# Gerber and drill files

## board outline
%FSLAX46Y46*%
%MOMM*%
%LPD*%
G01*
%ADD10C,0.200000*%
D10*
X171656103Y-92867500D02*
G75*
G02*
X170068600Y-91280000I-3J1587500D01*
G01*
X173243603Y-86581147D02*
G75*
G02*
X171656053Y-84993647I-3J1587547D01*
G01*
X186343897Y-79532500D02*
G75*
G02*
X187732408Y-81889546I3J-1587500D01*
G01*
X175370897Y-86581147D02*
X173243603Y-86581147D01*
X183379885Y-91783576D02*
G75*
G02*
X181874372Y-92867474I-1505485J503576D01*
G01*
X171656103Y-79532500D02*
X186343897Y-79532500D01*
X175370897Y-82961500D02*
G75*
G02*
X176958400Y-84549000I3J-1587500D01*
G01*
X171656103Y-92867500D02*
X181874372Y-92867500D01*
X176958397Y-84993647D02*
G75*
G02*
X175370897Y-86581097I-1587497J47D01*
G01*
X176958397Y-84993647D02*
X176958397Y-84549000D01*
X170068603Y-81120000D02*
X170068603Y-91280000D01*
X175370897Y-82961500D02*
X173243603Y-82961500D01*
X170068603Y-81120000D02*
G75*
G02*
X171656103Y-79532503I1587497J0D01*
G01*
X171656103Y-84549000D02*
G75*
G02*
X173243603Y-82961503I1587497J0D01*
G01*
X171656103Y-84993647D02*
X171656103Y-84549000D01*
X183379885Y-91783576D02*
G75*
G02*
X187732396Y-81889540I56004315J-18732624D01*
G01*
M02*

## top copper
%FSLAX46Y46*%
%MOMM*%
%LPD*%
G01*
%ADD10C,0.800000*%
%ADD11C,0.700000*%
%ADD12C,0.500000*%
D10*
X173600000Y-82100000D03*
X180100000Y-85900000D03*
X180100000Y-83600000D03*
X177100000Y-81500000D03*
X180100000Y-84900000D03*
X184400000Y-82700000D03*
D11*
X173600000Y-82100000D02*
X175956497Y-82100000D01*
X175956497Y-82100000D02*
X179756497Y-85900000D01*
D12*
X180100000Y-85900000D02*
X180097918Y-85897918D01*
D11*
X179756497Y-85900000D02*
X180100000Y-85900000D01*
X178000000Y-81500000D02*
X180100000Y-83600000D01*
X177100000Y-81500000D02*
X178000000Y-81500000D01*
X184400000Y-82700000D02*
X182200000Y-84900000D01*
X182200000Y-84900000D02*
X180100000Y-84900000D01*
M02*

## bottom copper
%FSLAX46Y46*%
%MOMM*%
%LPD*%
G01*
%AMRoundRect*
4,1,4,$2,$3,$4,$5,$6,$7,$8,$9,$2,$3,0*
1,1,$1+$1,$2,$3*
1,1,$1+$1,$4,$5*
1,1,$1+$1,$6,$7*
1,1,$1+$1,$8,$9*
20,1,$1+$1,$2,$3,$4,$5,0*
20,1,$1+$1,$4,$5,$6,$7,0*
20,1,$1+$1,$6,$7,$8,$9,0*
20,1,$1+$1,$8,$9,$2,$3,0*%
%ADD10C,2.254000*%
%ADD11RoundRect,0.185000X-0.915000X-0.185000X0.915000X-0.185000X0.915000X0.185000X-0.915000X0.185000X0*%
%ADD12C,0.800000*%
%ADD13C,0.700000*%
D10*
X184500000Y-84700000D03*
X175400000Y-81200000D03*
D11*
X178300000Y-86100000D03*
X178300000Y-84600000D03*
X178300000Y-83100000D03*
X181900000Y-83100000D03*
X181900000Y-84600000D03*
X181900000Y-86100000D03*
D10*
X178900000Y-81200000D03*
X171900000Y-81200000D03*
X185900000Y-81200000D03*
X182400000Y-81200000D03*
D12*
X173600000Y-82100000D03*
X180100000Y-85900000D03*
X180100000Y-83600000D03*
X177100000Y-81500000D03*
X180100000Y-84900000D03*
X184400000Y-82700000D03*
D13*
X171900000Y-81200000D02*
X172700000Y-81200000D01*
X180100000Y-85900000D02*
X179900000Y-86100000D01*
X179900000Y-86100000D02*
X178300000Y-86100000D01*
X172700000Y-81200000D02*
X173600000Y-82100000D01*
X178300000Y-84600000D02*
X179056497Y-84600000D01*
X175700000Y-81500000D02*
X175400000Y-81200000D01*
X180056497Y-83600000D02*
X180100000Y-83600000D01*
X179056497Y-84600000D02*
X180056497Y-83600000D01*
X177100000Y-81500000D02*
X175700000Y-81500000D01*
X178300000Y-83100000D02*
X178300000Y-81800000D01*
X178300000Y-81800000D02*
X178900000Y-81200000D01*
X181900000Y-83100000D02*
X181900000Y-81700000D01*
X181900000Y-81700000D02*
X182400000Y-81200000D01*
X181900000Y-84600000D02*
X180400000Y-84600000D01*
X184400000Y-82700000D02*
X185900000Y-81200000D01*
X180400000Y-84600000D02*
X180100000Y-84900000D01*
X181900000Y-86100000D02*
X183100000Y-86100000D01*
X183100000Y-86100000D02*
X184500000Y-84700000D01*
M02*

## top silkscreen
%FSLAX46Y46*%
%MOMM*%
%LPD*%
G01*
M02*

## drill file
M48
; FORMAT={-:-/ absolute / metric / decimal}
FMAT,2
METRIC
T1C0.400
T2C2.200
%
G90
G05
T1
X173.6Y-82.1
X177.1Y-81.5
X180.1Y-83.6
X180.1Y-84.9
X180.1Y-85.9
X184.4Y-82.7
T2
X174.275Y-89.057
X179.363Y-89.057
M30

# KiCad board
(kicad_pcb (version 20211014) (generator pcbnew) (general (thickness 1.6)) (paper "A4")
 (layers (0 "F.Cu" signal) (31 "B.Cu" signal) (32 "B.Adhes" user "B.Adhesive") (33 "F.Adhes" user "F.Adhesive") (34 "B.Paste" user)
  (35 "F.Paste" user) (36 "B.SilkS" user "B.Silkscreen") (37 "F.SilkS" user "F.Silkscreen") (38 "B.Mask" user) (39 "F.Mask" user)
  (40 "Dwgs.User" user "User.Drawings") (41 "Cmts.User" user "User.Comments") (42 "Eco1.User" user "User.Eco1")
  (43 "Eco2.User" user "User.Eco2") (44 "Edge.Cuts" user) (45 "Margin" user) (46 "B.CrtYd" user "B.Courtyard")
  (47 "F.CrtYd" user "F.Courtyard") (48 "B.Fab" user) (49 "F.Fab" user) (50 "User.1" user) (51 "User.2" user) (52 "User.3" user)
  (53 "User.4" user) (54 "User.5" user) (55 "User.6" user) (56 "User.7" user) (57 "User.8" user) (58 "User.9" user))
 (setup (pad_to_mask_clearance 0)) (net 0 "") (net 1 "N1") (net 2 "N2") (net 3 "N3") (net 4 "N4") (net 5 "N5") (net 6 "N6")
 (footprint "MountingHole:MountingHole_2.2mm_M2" (layer "F.Cu") (at 179.362966 89.0575)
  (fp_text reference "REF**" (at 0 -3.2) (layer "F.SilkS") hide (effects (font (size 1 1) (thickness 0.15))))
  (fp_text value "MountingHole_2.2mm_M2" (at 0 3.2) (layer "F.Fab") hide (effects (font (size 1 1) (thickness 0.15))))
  (pad "" np_thru_hole circle (at 0 0) (size 2.2 2.2) (drill 2.2) (layers *.Cu *.Mask)))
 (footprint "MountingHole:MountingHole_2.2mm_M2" (layer "F.Cu") (at 174.275478 89.0575)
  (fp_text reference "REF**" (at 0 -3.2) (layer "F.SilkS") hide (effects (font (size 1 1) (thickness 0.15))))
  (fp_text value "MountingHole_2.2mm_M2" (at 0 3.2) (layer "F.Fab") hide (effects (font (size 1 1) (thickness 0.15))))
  (pad "" np_thru_hole circle (at 0 0) (size 2.2 2.2) (drill 2.2) (layers *.Cu *.Mask)))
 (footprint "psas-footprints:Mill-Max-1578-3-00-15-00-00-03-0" (layer "B.Cu") (at 184.5 84.7 180)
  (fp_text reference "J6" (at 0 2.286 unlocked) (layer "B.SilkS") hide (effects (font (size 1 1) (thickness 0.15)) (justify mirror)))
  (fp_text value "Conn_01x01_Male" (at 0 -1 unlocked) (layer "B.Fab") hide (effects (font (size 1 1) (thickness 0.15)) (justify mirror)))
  (pad "1" smd circle (at 0 0 180) (size 2.254 2.254) (layers "B.Cu" "B.Paste" "B.Mask") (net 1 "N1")))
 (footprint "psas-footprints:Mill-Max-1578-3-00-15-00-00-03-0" (layer "B.Cu") (at 175.4 81.2 180)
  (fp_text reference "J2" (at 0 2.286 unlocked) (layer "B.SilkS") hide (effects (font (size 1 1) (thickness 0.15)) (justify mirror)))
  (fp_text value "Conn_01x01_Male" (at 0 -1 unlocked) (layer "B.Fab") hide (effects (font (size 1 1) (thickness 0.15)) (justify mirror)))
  (pad "1" smd circle (at 0 0 180) (size 2.254 2.254) (layers "B.Cu" "B.Paste" "B.Mask") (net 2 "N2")))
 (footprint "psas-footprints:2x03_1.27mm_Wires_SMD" (layer "B.Cu") (at 180.1 84.6)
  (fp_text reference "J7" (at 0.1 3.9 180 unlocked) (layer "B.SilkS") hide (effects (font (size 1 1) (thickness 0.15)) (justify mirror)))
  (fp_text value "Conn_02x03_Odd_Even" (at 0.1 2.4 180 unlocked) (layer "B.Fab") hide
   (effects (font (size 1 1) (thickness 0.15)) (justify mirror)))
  (pad "1" smd roundrect (at -1.8 1.5) (size 2.2 0.74) (layers "B.Cu" "B.Paste" "B.Mask") (roundrect_rratio 0.25) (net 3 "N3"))
  (pad "2" smd roundrect (at -1.8 0) (size 2.2 0.74) (layers "B.Cu" "B.Paste" "B.Mask") (roundrect_rratio 0.25) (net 2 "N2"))
  (pad "3" smd roundrect (at -1.8 -1.5) (size 2.2 0.74) (layers "B.Cu" "B.Paste" "B.Mask") (roundrect_rratio 0.25) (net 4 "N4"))
  (pad "4" smd roundrect (at 1.8 -1.5) (size 2.2 0.74) (layers "B.Cu" "B.Paste" "B.Mask") (roundrect_rratio 0.25) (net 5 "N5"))
  (pad "5" smd roundrect (at 1.8 0) (size 2.2 0.74) (layers "B.Cu" "B.Paste" "B.Mask") (roundrect_rratio 0.25) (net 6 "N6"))
  (pad "6" smd roundrect (at 1.8 1.5) (size 2.2 0.74) (layers "B.Cu" "B.Paste" "B.Mask") (roundrect_rratio 0.25) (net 1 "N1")))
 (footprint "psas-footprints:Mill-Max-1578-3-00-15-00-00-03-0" (layer "B.Cu") (at 178.9 81.2 180)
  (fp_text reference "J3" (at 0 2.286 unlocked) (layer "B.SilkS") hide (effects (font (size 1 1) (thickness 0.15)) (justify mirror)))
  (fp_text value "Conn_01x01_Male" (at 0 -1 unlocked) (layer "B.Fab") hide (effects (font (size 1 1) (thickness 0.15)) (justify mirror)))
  (pad "1" smd circle (at 0 0 180) (size 2.254 2.254) (layers "B.Cu" "B.Paste" "B.Mask") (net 4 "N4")))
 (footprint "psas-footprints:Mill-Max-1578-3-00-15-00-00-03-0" (layer "B.Cu") (at 171.9 81.2 180)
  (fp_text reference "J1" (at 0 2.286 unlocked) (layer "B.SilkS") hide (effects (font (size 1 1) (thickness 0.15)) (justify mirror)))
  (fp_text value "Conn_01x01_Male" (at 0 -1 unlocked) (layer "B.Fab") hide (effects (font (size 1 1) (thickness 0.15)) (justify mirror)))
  (pad "1" smd circle (at 0 0 180) (size 2.254 2.254) (layers "B.Cu" "B.Paste" "B.Mask") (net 3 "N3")))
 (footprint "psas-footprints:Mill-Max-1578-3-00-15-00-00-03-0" (layer "B.Cu") (at 185.9 81.2 180)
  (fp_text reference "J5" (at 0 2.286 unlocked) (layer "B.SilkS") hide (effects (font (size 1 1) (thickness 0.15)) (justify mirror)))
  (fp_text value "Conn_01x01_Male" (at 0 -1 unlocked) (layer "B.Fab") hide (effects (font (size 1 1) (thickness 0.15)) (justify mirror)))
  (pad "1" smd circle (at 0 0 180) (size 2.254 2.254) (layers "B.Cu" "B.Paste" "B.Mask") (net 6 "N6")))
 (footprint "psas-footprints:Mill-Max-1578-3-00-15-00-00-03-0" (layer "B.Cu") (at 182.4 81.2 180)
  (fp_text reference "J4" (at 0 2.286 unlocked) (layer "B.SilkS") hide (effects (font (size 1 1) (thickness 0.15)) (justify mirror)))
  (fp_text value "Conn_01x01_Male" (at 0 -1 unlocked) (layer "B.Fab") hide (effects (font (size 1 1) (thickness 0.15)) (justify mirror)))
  (pad "1" smd circle (at 0 0 180) (size 2.254 2.254) (layers "B.Cu" "B.Paste" "B.Mask") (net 5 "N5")))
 (gr_arc (start 171.656103 92.8675) (mid 170.533571 92.402532) (end 170.068603 91.28) (layer "Edge.Cuts") (width 0.2))
 (gr_arc (start 173.243603 86.581147) (mid 172.121071 86.116179) (end 171.656103 84.993647) (layer "Edge.Cuts") (width 0.2))
 (gr_arc (start 186.343897 79.5325) (mid 187.711707 80.314238) (end 187.732406 81.889545) (layer "Edge.Cuts") (width 0.2))
 (gr_line (start 175.370897 86.581147) (end 173.243603 86.581147) (layer "Edge.Cuts") (width 0.2))
 (gr_arc (start 183.379885 91.783576) (mid 182.801931 92.568329) (end 181.874372 92.8675) (layer "Edge.Cuts") (width 0.2))
 (gr_line (start 171.656103 79.5325) (end 186.343897 79.5325) (layer "Edge.Cuts") (width 0.2))
 (gr_arc (start 175.370897 82.9615) (mid 176.493429 83.426468) (end 176.958397 84.549) (layer "Edge.Cuts") (width 0.2))
 (gr_line (start 171.656103 92.8675) (end 181.874372 92.8675) (layer "Edge.Cuts") (width 0.2))
 (gr_arc (start 176.958397 84.993647) (mid 176.493429 86.116179) (end 175.370897 86.581147) (layer "Edge.Cuts") (width 0.2))
 (gr_line (start 176.958397 84.993647) (end 176.958397 84.549) (layer "Edge.Cuts") (width 0.2))
 (gr_line (start 170.068603 81.12) (end 170.068603 91.28) (layer "Edge.Cuts") (width 0.2))
 (gr_line (start 175.370897 82.9615) (end 173.243603 82.9615) (layer "Edge.Cuts") (width 0.2))
 (gr_arc (start 170.068603 81.12) (mid 170.533571 79.997468) (end 171.656103 79.5325) (layer "Edge.Cuts") (width 0.2))
 (gr_arc (start 171.656103 84.549) (mid 172.121071 83.426468) (end 173.243603 82.9615) (layer "Edge.Cuts") (width 0.2))
 (gr_line (start 171.656103 84.993647) (end 171.656103 84.549) (layer "Edge.Cuts") (width 0.2))
 (gr_arc (start 183.379885 91.783576) (mid 185.329298 86.736767) (end 187.732406 81.889545) (layer "Edge.Cuts") (width 0.2))
 (segment (start 173.6 82.1) (end 175.956497 82.1) (width 0.7) (layer "F.Cu") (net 3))
 (segment (start 175.956497 82.1) (end 179.756497 85.9) (width 0.7) (layer "F.Cu") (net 3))
 (segment (start 180.1 85.9) (end 180.097918 85.897918) (width 0.5) (layer "F.Cu") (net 3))
 (segment (start 179.756497 85.9) (end 180.1 85.9) (width 0.7) (layer "F.Cu") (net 3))
 (via (at 173.6 82.1) (size 0.8) (drill 0.4) (layers "F.Cu" "B.Cu") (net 3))
 (via (at 180.1 85.9) (size 0.8) (drill 0.4) (layers "F.Cu" "B.Cu") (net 3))
 (segment (start 171.9 81.2) (end 172.7 81.2) (width 0.7) (layer "B.Cu") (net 3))
 (segment (start 180.1 85.9) (end 179.9 86.1) (width 0.7) (layer "B.Cu") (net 3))
 (segment (start 179.9 86.1) (end 178.3 86.1) (width 0.7) (layer "B.Cu") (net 3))
 (segment (start 172.7 81.2) (end 173.6 82.1) (width 0.7) (layer "B.Cu") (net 3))
 (segment (start 178 81.5) (end 180.1 83.6) (width 0.7) (layer "F.Cu") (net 2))
 (segment (start 177.1 81.5) (end 178 81.5) (width 0.7) (layer "F.Cu") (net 2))
 (via (at 180.1 83.6) (size 0.8) (drill 0.4) (layers "F.Cu" "B.Cu") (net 2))
 (via (at 177.1 81.5) (size 0.8) (drill 0.4) (layers "F.Cu" "B.Cu") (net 2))
 (segment (start 178.3 84.6) (end 179.056497 84.6) (width 0.7) (layer "B.Cu") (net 2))
 (segment (start 175.7 81.5) (end 175.4 81.2) (width 0.7) (layer "B.Cu") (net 2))
 (segment (start 180.056497 83.6) (end 180.1 83.6) (width 0.7) (layer "B.Cu") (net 2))
 (segment (start 179.056497 84.6) (end 180.056497 83.6) (width 0.7) (layer "B.Cu") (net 2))
 (segment (start 177.1 81.5) (end 175.7 81.5) (width 0.7) (layer "B.Cu") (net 2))
 (segment (start 178.3 83.1) (end 178.3 81.8) (width 0.7) (layer "B.Cu") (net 4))
 (segment (start 178.3 81.8) (end 178.9 81.2) (width 0.7) (layer "B.Cu") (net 4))
 (segment (start 181.9 83.1) (end 181.9 81.7) (width 0.7) (layer "B.Cu") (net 5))
 (segment (start 181.9 81.7) (end 182.4 81.2) (width 0.7) (layer "B.Cu") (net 5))
 (segment (start 184.4 82.7) (end 182.2 84.9) (width 0.7) (layer "F.Cu") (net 6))
 (segment (start 182.2 84.9) (end 180.1 84.9) (width 0.7) (layer "F.Cu") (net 6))
 (via (at 180.1 84.9) (size 0.8) (drill 0.4) (layers "F.Cu" "B.Cu") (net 6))
 (via (at 184.4 82.7) (size 0.8) (drill 0.4) (layers "F.Cu" "B.Cu") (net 6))
 (segment (start 181.9 84.6) (end 180.4 84.6) (width 0.7) (layer "B.Cu") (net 6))
 (segment (start 184.4 82.7) (end 185.9 81.2) (width 0.7) (layer "B.Cu") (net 6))
 (segment (start 180.4 84.6) (end 180.1 84.9) (width 0.7) (layer "B.Cu") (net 6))
 (segment (start 181.9 86.1) (end 183.1 86.1) (width 0.7) (layer "B.Cu") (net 1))
 (segment (start 183.1 86.1) (end 184.5 84.7) (width 0.7) (layer "B.Cu") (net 1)))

